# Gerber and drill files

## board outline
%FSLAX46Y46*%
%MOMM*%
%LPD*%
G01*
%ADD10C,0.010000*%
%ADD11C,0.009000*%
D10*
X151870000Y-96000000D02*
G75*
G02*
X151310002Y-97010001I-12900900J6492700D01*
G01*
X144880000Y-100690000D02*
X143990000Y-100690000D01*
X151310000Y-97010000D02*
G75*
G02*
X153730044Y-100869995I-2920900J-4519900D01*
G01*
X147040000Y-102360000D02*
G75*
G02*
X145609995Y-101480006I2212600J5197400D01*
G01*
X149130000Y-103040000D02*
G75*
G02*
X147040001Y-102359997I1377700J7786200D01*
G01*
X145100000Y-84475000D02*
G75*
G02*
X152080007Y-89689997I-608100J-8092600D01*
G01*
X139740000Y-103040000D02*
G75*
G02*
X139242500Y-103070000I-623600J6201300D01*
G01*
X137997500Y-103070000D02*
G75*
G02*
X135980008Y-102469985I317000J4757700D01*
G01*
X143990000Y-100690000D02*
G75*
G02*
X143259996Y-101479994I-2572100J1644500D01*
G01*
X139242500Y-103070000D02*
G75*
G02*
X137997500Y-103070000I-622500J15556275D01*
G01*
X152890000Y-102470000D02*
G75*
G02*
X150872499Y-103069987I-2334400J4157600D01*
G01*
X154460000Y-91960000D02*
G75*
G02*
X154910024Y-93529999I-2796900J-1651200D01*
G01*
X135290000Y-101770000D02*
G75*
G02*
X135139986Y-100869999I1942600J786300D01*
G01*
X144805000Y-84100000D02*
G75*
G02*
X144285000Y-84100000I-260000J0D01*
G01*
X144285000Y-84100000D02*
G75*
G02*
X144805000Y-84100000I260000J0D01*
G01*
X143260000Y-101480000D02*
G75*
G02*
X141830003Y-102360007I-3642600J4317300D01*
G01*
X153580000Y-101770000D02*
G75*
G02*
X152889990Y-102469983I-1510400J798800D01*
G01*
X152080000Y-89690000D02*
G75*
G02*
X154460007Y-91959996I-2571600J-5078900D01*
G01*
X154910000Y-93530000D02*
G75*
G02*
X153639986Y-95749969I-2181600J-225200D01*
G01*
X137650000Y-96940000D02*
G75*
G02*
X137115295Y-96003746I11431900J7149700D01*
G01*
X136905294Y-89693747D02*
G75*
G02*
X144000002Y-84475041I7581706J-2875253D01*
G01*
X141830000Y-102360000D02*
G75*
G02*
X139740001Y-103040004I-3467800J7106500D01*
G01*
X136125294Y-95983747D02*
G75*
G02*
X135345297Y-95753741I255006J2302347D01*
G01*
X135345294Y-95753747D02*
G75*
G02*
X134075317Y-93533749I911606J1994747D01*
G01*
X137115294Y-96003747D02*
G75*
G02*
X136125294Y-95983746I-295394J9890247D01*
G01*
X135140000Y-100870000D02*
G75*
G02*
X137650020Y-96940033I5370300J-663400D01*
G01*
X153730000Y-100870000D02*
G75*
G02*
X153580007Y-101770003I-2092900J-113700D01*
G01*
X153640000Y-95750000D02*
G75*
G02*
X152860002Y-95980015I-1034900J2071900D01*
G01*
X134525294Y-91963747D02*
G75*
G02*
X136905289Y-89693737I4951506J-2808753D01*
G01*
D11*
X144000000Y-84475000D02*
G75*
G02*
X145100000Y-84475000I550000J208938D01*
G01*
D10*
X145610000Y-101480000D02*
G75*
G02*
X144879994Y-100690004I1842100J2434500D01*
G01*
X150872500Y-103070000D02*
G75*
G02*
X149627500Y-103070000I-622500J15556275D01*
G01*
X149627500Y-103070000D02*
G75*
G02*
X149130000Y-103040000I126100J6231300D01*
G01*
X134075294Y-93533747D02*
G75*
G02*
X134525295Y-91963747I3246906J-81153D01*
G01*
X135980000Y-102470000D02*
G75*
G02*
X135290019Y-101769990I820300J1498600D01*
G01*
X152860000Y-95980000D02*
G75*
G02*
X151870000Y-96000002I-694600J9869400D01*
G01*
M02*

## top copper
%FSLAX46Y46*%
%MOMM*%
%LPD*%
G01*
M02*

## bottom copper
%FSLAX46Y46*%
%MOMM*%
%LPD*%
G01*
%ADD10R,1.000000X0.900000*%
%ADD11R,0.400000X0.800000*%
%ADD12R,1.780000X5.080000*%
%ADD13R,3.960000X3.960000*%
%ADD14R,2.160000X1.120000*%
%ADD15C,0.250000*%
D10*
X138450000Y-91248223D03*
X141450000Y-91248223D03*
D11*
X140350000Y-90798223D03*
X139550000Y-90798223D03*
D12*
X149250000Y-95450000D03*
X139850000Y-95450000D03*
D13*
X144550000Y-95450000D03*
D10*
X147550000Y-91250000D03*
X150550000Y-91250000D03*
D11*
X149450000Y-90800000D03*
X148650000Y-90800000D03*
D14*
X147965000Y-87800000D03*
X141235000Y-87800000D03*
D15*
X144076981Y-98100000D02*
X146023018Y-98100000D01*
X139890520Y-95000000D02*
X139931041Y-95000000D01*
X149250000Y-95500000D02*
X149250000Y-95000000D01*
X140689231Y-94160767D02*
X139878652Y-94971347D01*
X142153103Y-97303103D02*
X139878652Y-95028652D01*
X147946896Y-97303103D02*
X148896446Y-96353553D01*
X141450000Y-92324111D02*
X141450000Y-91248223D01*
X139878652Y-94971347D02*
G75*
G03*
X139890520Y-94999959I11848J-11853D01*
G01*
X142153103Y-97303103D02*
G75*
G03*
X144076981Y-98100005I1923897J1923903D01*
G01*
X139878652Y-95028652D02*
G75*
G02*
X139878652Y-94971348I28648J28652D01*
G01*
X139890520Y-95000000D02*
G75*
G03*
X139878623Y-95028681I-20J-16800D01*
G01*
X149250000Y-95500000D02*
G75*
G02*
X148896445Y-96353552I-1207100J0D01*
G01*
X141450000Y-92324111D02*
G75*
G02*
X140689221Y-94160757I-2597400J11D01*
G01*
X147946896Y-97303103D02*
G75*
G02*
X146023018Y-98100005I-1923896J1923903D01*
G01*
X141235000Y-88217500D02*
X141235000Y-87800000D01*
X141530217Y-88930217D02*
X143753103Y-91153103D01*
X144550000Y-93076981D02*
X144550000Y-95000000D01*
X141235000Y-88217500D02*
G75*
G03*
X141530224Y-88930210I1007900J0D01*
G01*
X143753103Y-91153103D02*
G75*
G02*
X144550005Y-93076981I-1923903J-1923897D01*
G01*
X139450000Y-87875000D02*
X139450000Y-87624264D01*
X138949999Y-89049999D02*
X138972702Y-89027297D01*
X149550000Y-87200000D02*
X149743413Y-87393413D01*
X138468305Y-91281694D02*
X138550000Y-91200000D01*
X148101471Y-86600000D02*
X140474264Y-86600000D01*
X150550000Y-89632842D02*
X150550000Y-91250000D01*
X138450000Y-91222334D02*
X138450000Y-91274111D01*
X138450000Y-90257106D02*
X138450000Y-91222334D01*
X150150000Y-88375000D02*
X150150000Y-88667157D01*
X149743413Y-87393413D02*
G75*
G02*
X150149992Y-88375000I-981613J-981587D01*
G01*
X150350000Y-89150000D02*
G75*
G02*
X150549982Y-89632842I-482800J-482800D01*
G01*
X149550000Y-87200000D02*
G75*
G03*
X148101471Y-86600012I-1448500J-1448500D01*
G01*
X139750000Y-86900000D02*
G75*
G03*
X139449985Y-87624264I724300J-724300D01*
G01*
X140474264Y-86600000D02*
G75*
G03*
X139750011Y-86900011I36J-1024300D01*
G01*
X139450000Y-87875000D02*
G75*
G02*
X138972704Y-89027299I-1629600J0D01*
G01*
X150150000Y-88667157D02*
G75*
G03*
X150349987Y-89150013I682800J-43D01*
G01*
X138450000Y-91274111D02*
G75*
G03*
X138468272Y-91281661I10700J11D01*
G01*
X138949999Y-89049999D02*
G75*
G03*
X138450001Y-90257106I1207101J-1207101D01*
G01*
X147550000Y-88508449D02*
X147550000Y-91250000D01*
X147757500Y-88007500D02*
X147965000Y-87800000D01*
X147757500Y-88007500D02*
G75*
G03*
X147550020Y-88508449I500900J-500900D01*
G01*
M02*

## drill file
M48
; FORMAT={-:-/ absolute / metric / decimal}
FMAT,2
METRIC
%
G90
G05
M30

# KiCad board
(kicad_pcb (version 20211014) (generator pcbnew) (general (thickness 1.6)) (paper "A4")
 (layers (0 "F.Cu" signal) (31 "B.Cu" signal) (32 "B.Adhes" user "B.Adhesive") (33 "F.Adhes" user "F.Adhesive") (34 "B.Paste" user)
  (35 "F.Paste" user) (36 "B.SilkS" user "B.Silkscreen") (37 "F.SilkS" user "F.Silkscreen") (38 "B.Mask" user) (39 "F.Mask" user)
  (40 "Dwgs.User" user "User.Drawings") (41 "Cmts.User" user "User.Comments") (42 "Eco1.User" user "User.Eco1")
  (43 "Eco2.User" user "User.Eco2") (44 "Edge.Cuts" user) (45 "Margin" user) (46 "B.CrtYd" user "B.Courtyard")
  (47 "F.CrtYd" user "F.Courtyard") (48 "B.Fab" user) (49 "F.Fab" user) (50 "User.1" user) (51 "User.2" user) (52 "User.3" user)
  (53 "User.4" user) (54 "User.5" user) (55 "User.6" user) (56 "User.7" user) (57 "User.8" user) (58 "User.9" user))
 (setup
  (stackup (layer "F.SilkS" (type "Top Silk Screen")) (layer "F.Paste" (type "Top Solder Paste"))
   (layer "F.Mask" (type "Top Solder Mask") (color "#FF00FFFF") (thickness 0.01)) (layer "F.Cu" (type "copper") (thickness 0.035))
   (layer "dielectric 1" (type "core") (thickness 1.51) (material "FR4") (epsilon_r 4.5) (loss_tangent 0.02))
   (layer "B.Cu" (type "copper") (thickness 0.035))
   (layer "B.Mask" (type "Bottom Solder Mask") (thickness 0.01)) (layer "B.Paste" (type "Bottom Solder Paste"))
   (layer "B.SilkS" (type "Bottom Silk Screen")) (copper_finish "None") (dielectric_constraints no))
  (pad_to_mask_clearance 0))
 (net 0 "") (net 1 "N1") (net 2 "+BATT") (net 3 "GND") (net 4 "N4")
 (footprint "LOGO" (layer "F.Cu") (at 144.51 93.77)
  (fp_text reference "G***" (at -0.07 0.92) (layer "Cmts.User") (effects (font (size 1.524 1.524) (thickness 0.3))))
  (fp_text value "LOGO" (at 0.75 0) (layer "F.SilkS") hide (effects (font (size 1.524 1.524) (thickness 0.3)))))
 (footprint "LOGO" (layer "F.Cu") (at 144.51 93.77)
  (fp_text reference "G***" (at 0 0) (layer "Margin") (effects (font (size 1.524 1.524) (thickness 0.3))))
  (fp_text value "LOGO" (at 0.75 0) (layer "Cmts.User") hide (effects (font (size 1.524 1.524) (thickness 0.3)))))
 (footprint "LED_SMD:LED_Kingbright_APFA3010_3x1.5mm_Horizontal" (layer "B.Cu") (at 139.95 91.248223)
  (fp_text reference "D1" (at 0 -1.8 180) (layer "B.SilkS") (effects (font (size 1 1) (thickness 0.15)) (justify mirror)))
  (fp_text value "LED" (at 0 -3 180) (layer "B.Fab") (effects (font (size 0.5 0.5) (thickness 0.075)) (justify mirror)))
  (pad "1" smd rect (at -1.5 0) (size 1 0.9) (layers "B.Cu" "B.Paste" "B.Mask") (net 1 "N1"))
  (pad "2" smd rect (at 1.5 0) (size 1 0.9) (layers "B.Cu" "B.Paste" "B.Mask") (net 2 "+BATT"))
  (pad "3" smd rect (at 0.4 -0.45) (size 0.4 0.8) (layers "B.Cu" "B.Paste" "B.Mask"))
  (pad "4" smd rect (at -0.4 -0.45) (size 0.4 0.8) (layers "B.Cu" "B.Paste" "B.Mask")))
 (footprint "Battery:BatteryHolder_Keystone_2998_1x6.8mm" (layer "B.Cu") (at 144.55 95.45 180)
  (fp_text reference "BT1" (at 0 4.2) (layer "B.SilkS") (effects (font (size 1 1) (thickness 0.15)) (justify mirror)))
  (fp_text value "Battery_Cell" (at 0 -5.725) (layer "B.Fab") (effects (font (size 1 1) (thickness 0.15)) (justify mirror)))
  (pad "1" smd rect (at -4.7 0 180) (size 1.78 5.08) (layers "B.Cu" "B.Paste" "B.Mask") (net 2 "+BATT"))
  (pad "1" smd rect (at 4.7 0 180) (size 1.78 5.08) (layers "B.Cu" "B.Paste" "B.Mask") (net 2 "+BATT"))
  (pad "2" smd rect (at 0 0 180) (size 3.96 3.96) (layers "B.Cu" "B.Paste" "B.Mask") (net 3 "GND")))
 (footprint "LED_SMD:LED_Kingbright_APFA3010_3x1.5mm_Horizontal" (layer "B.Cu") (at 149.05 91.25)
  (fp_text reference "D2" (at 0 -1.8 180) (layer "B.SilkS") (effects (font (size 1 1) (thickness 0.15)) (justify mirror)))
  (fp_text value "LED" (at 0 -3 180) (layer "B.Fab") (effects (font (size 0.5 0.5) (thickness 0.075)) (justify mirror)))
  (pad "1" smd rect (at -1.5 0) (size 1 0.9) (layers "B.Cu" "B.Paste" "B.Mask") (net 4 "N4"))
  (pad "2" smd rect (at 1.5 0) (size 1 0.9) (layers "B.Cu" "B.Paste" "B.Mask") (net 1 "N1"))
  (pad "3" smd rect (at 0.4 -0.45) (size 0.4 0.8) (layers "B.Cu" "B.Paste" "B.Mask"))
  (pad "4" smd rect (at -0.4 -0.45) (size 0.4 0.8) (layers "B.Cu" "B.Paste" "B.Mask")))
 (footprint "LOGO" (layer "B.Cu") (at 144.51 93.77 180)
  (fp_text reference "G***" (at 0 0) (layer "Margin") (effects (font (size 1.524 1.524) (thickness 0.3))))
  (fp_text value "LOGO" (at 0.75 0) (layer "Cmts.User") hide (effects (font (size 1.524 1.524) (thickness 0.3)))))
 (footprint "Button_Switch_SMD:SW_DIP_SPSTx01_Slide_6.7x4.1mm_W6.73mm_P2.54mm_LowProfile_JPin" (layer "B.Cu") (at 144.6 87.8 180)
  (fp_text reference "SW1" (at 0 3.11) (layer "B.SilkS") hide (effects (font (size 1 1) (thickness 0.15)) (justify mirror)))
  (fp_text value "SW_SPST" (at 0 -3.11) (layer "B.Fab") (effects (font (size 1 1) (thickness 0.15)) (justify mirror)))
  (pad "1" smd rect (at -3.365 0 180) (size 2.16 1.12) (layers "B.Cu" "B.Paste" "B.Mask") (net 4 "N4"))
  (pad "2" smd rect (at 3.365 0 180) (size 2.16 1.12) (layers "B.Cu" "B.Paste" "B.Mask") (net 3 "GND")))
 (gr_arc (start 151.87 96) (mid 151.600099 96.5106) (end 151.31 97.01) (layer "Edge.Cuts") (width 0.01))
 (gr_line (start 144.88 100.69) (end 143.99 100.69) (layer "Edge.Cuts") (width 0.01))
 (gr_arc (start 151.31 97.01) (mid 152.948615 98.671276) (end 153.73 100.87) (layer "Edge.Cuts") (width 0.01))
 (gr_arc (start 147.04 102.36) (mid 146.29212 101.973429) (end 145.61 101.48) (layer "Edge.Cuts") (width 0.01))
 (gr_arc (start 149.13 103.04) (mid 148.061259 102.77297) (end 147.04 102.36) (layer "Edge.Cuts") (width 0.01))
 (gr_arc (start 145.1 84.475) (mid 149.349208 86.066341) (end 152.08 89.69) (layer "Edge.Cuts") (width 0.01))
 (gr_arc (start 139.74 103.04) (mid 139.49155 103.059975) (end 139.2425 103.07) (layer "Edge.Cuts") (width 0.01))
 (gr_arc (start 137.9975 103.07) (mid 136.95523 102.882711) (end 135.98 102.47) (layer "Edge.Cuts") (width 0.01))
 (gr_arc (start 143.99 100.69) (mid 143.660067 101.117404) (end 143.26 101.48) (layer "Edge.Cuts") (width 0.01))
 (gr_arc (start 139.2425 103.07) (mid 138.62 103.08245) (end 137.9975 103.07) (layer "Edge.Cuts") (width 0.01))
 (gr_arc (start 152.89 102.47) (mid 151.91477 102.882714) (end 150.8725 103.07) (layer "Edge.Cuts") (width 0.01))
 (gr_arc (start 154.46 91.96) (mid 154.785294 92.716253) (end 154.91 93.53) (layer "Edge.Cuts") (width 0.01))
 (gr_arc (start 135.29 101.77) (mid 135.165425 101.328262) (end 135.14 100.87) (layer "Edge.Cuts") (width 0.01))
 (gr_circle (center 144.545 84.1) (end 144.805 84.1) (layer "Edge.Cuts") (width 0.01) (fill none))
 (gr_arc (start 143.26 101.48) (mid 142.57788 101.97343) (end 141.83 102.36) (layer "Edge.Cuts") (width 0.01))
 (gr_arc (start 153.58 101.77) (mid 153.286422 102.170687) (end 152.89 102.47) (layer "Edge.Cuts") (width 0.01))
 (gr_arc (start 152.08 89.69) (mid 153.4375 90.649376) (end 154.46 91.96) (layer "Edge.Cuts") (width 0.01))
 (gr_arc (start 154.91 93.53) (mid 154.632101 94.844288) (end 153.64 95.75) (layer "Edge.Cuts") (width 0.01))
 (gr_arc (start 137.65 96.94) (mid 137.373285 96.47722) (end 137.115294 96.003747) (layer "Edge.Cuts") (width 0.01))
 (gr_arc (start 136.905294 89.693747) (mid 139.682339 86.037166) (end 144 84.475) (layer "Edge.Cuts") (width 0.01))
 (gr_arc (start 141.83 102.36) (mid 140.808741 102.772967) (end 139.74 103.04) (layer "Edge.Cuts") (width 0.01))
 (gr_arc (start 136.125294 95.983747) (mid 135.725123 95.903243) (end 135.345294 95.753747) (layer "Edge.Cuts") (width 0.01))
 (gr_arc (start 135.345294 95.753747) (mid 134.353193 94.848035) (end 134.075294 93.533747) (layer "Edge.Cuts") (width 0.01))
 (gr_arc (start 137.115294 96.003747) (mid 136.620044 96.006139) (end 136.125294 95.983747) (layer "Edge.Cuts") (width 0.01))
 (gr_arc (start 135.14 100.87) (mid 135.94994 98.620751) (end 137.65 96.94) (layer "Edge.Cuts") (width 0.01))
 (gr_arc (start 153.73 100.87) (mid 153.704567 101.328262) (end 153.58 101.77) (layer "Edge.Cuts") (width 0.01))
 (gr_arc (start 153.64 95.75) (mid 153.260174 95.899503) (end 152.86 95.98) (layer "Edge.Cuts") (width 0.01))
 (gr_arc (start 134.525294 91.963747) (mid 135.547787 90.653122) (end 136.905294 89.693747) (layer "Edge.Cuts") (width 0.01))
 (gr_arc (start 144 84.475) (mid 144.55 83.677713) (end 145.1 84.475) (layer "Edge.Cuts") (width 0.009))
 (gr_arc (start 145.61 101.48) (mid 145.209933 101.117404) (end 144.88 100.69) (layer "Edge.Cuts") (width 0.01))
 (gr_arc (start 150.8725 103.07) (mid 150.25 103.08245) (end 149.6275 103.07) (layer "Edge.Cuts") (width 0.01))
 (gr_arc (start 149.6275 103.07) (mid 149.37845 103.059975) (end 149.13 103.04) (layer "Edge.Cuts") (width 0.01))
 (gr_arc (start 134.075294 93.533747) (mid 134.2 92.72) (end 134.525294 91.963747) (layer "Edge.Cuts") (width 0.01))
 (gr_arc (start 135.98 102.47) (mid 135.58357 102.170693) (end 135.29 101.77) (layer "Edge.Cuts") (width 0.01))
 (gr_arc (start 152.86 95.98) (mid 152.36525 96.002393) (end 151.87 96) (layer "Edge.Cuts") (width 0.01))
 (segment (start 144.076981 98.1) (end 146.023018 98.1) (width 0.25) (layer "B.Cu") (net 2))
 (segment (start 139.89052 95) (end 139.931041 95) (width 0.25) (layer "B.Cu") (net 2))
 (segment (start 149.25 95.5) (end 149.25 95) (width 0.25) (layer "B.Cu") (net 2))
 (segment (start 140.689231 94.160767) (end 139.878652 94.971347) (width 0.25) (layer "B.Cu") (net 2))
 (segment (start 142.153103 97.303103) (end 139.878652 95.028652) (width 0.25) (layer "B.Cu") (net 2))
 (segment (start 147.946896 97.303103) (end 148.896446 96.353553) (width 0.25) (layer "B.Cu") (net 2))
 (segment (start 141.45 92.324111) (end 141.45 91.248223) (width 0.25) (layer "B.Cu") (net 2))
 (arc (start 139.878652 94.971347) (mid 139.875013 94.989638) (end 139.89052 95) (width 0.25) (layer "B.Cu") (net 2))
 (arc (start 142.153103 97.303103) (mid 143.035786 97.892893) (end 144.076981 98.1) (width 0.25) (layer "B.Cu") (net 2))
 (arc (start 139.878652 95.028652) (mid 139.866783 94.999999) (end 139.878652 94.971347) (width 0.25) (layer "B.Cu") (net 2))
 (arc (start 139.89052 95) (mid 139.875013 95.010361) (end 139.878652 95.028652) (width 0.25) (layer "B.Cu") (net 2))
 (arc (start 149.25 95.5) (mid 149.158114 95.961939) (end 148.896446 96.353553) (width 0.25) (layer "B.Cu") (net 2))
 (arc (start 141.45 92.324111) (mid 141.252282 93.318102) (end 140.689231 94.160767) (width 0.25) (layer "B.Cu") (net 2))
 (arc (start 147.946896 97.303103) (mid 147.064213 97.892893) (end 146.023018 98.1) (width 0.25) (layer "B.Cu") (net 2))
 (segment (start 141.235 88.2175) (end 141.235 87.8) (width 0.25) (layer "B.Cu") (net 3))
 (segment (start 141.530217 88.930217) (end 143.753103 91.153103) (width 0.25) (layer "B.Cu") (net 3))
 (segment (start 144.55 93.076981) (end 144.55 95) (width 0.25) (layer "B.Cu") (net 3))
 (arc (start 141.235 88.2175) (mid 141.311724 88.603219) (end 141.530217 88.930217) (width 0.25) (layer "B.Cu") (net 3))
 (arc (start 143.753103 91.153103) (mid 144.342893 92.035786) (end 144.55 93.076981) (width 0.25) (layer "B.Cu") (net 3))
 (segment (start 139.45 87.875) (end 139.45 87.624264) (width 0.25) (layer "B.Cu") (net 1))
 (segment (start 138.949999 89.049999) (end 138.972702 89.027297) (width 0.25) (layer "B.Cu") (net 1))
 (segment (start 149.55 87.2) (end 149.743413 87.393413) (width 0.25) (layer "B.Cu") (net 1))
 (segment (start 138.468305 91.281694) (end 138.55 91.2) (width 0.25) (layer "B.Cu") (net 1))
 (segment (start 148.101471 86.6) (end 140.474264 86.6) (width 0.25) (layer "B.Cu") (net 1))
 (segment (start 150.55 89.632842) (end 150.55 91.25) (width 0.25) (layer "B.Cu") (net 1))
 (segment (start 138.45 91.222334) (end 138.45 91.274111) (width 0.25) (layer "B.Cu") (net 1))
 (segment (start 138.45 90.257106) (end 138.45 91.222334) (width 0.25) (layer "B.Cu") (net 1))
 (segment (start 150.15 88.375) (end 150.15 88.667157) (width 0.25) (layer "B.Cu") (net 1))
 (arc (start 149.743413 87.393413) (mid 150.044331 87.843769) (end 150.15 88.375) (width 0.25) (layer "B.Cu") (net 1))
 (arc (start 150.35 89.15) (mid 150.498021 89.371529) (end 150.55 89.632842) (width 0.25) (layer "B.Cu") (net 1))
 (arc (start 149.55 87.2) (mid 148.885409 86.755934) (end 148.101471 86.6) (width 0.25) (layer "B.Cu") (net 1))
 (arc (start 139.75 86.9) (mid 139.527967 87.232295) (end 139.45 87.624264) (width 0.25) (layer "B.Cu") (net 1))
 (arc (start 140.474264 86.6) (mid 140.082295 86.677967) (end 139.75 86.9) (width 0.25) (layer "B.Cu") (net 1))
 (arc (start 139.45 87.875) (mid 139.325954 88.498618) (end 138.972702 89.027297) (width 0.25) (layer "B.Cu") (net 1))
 (arc (start 150.15 88.667157) (mid 150.201978 88.928469) (end 150.35 89.15) (width 0.25) (layer "B.Cu") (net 1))
 (arc (start 138.45 91.274111) (mid 138.456619 91.284018) (end 138.468305 91.281694) (width 0.25) (layer "B.Cu") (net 1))
 (arc (start 138.949999 89.049999) (mid 138.579945 89.603824) (end 138.45 90.257106) (width 0.25) (layer "B.Cu") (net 1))
 (segment (start 147.55 88.508449) (end 147.55 91.25) (width 0.25) (layer "B.Cu") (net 4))
 (segment (start 147.7575 88.0075) (end 147.965 87.8) (width 0.25) (layer "B.Cu") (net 4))
 (arc (start 147.7575 88.0075) (mid 147.603927 88.237337) (end 147.55 88.508449) (width 0.25) (layer "B.Cu") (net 4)))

